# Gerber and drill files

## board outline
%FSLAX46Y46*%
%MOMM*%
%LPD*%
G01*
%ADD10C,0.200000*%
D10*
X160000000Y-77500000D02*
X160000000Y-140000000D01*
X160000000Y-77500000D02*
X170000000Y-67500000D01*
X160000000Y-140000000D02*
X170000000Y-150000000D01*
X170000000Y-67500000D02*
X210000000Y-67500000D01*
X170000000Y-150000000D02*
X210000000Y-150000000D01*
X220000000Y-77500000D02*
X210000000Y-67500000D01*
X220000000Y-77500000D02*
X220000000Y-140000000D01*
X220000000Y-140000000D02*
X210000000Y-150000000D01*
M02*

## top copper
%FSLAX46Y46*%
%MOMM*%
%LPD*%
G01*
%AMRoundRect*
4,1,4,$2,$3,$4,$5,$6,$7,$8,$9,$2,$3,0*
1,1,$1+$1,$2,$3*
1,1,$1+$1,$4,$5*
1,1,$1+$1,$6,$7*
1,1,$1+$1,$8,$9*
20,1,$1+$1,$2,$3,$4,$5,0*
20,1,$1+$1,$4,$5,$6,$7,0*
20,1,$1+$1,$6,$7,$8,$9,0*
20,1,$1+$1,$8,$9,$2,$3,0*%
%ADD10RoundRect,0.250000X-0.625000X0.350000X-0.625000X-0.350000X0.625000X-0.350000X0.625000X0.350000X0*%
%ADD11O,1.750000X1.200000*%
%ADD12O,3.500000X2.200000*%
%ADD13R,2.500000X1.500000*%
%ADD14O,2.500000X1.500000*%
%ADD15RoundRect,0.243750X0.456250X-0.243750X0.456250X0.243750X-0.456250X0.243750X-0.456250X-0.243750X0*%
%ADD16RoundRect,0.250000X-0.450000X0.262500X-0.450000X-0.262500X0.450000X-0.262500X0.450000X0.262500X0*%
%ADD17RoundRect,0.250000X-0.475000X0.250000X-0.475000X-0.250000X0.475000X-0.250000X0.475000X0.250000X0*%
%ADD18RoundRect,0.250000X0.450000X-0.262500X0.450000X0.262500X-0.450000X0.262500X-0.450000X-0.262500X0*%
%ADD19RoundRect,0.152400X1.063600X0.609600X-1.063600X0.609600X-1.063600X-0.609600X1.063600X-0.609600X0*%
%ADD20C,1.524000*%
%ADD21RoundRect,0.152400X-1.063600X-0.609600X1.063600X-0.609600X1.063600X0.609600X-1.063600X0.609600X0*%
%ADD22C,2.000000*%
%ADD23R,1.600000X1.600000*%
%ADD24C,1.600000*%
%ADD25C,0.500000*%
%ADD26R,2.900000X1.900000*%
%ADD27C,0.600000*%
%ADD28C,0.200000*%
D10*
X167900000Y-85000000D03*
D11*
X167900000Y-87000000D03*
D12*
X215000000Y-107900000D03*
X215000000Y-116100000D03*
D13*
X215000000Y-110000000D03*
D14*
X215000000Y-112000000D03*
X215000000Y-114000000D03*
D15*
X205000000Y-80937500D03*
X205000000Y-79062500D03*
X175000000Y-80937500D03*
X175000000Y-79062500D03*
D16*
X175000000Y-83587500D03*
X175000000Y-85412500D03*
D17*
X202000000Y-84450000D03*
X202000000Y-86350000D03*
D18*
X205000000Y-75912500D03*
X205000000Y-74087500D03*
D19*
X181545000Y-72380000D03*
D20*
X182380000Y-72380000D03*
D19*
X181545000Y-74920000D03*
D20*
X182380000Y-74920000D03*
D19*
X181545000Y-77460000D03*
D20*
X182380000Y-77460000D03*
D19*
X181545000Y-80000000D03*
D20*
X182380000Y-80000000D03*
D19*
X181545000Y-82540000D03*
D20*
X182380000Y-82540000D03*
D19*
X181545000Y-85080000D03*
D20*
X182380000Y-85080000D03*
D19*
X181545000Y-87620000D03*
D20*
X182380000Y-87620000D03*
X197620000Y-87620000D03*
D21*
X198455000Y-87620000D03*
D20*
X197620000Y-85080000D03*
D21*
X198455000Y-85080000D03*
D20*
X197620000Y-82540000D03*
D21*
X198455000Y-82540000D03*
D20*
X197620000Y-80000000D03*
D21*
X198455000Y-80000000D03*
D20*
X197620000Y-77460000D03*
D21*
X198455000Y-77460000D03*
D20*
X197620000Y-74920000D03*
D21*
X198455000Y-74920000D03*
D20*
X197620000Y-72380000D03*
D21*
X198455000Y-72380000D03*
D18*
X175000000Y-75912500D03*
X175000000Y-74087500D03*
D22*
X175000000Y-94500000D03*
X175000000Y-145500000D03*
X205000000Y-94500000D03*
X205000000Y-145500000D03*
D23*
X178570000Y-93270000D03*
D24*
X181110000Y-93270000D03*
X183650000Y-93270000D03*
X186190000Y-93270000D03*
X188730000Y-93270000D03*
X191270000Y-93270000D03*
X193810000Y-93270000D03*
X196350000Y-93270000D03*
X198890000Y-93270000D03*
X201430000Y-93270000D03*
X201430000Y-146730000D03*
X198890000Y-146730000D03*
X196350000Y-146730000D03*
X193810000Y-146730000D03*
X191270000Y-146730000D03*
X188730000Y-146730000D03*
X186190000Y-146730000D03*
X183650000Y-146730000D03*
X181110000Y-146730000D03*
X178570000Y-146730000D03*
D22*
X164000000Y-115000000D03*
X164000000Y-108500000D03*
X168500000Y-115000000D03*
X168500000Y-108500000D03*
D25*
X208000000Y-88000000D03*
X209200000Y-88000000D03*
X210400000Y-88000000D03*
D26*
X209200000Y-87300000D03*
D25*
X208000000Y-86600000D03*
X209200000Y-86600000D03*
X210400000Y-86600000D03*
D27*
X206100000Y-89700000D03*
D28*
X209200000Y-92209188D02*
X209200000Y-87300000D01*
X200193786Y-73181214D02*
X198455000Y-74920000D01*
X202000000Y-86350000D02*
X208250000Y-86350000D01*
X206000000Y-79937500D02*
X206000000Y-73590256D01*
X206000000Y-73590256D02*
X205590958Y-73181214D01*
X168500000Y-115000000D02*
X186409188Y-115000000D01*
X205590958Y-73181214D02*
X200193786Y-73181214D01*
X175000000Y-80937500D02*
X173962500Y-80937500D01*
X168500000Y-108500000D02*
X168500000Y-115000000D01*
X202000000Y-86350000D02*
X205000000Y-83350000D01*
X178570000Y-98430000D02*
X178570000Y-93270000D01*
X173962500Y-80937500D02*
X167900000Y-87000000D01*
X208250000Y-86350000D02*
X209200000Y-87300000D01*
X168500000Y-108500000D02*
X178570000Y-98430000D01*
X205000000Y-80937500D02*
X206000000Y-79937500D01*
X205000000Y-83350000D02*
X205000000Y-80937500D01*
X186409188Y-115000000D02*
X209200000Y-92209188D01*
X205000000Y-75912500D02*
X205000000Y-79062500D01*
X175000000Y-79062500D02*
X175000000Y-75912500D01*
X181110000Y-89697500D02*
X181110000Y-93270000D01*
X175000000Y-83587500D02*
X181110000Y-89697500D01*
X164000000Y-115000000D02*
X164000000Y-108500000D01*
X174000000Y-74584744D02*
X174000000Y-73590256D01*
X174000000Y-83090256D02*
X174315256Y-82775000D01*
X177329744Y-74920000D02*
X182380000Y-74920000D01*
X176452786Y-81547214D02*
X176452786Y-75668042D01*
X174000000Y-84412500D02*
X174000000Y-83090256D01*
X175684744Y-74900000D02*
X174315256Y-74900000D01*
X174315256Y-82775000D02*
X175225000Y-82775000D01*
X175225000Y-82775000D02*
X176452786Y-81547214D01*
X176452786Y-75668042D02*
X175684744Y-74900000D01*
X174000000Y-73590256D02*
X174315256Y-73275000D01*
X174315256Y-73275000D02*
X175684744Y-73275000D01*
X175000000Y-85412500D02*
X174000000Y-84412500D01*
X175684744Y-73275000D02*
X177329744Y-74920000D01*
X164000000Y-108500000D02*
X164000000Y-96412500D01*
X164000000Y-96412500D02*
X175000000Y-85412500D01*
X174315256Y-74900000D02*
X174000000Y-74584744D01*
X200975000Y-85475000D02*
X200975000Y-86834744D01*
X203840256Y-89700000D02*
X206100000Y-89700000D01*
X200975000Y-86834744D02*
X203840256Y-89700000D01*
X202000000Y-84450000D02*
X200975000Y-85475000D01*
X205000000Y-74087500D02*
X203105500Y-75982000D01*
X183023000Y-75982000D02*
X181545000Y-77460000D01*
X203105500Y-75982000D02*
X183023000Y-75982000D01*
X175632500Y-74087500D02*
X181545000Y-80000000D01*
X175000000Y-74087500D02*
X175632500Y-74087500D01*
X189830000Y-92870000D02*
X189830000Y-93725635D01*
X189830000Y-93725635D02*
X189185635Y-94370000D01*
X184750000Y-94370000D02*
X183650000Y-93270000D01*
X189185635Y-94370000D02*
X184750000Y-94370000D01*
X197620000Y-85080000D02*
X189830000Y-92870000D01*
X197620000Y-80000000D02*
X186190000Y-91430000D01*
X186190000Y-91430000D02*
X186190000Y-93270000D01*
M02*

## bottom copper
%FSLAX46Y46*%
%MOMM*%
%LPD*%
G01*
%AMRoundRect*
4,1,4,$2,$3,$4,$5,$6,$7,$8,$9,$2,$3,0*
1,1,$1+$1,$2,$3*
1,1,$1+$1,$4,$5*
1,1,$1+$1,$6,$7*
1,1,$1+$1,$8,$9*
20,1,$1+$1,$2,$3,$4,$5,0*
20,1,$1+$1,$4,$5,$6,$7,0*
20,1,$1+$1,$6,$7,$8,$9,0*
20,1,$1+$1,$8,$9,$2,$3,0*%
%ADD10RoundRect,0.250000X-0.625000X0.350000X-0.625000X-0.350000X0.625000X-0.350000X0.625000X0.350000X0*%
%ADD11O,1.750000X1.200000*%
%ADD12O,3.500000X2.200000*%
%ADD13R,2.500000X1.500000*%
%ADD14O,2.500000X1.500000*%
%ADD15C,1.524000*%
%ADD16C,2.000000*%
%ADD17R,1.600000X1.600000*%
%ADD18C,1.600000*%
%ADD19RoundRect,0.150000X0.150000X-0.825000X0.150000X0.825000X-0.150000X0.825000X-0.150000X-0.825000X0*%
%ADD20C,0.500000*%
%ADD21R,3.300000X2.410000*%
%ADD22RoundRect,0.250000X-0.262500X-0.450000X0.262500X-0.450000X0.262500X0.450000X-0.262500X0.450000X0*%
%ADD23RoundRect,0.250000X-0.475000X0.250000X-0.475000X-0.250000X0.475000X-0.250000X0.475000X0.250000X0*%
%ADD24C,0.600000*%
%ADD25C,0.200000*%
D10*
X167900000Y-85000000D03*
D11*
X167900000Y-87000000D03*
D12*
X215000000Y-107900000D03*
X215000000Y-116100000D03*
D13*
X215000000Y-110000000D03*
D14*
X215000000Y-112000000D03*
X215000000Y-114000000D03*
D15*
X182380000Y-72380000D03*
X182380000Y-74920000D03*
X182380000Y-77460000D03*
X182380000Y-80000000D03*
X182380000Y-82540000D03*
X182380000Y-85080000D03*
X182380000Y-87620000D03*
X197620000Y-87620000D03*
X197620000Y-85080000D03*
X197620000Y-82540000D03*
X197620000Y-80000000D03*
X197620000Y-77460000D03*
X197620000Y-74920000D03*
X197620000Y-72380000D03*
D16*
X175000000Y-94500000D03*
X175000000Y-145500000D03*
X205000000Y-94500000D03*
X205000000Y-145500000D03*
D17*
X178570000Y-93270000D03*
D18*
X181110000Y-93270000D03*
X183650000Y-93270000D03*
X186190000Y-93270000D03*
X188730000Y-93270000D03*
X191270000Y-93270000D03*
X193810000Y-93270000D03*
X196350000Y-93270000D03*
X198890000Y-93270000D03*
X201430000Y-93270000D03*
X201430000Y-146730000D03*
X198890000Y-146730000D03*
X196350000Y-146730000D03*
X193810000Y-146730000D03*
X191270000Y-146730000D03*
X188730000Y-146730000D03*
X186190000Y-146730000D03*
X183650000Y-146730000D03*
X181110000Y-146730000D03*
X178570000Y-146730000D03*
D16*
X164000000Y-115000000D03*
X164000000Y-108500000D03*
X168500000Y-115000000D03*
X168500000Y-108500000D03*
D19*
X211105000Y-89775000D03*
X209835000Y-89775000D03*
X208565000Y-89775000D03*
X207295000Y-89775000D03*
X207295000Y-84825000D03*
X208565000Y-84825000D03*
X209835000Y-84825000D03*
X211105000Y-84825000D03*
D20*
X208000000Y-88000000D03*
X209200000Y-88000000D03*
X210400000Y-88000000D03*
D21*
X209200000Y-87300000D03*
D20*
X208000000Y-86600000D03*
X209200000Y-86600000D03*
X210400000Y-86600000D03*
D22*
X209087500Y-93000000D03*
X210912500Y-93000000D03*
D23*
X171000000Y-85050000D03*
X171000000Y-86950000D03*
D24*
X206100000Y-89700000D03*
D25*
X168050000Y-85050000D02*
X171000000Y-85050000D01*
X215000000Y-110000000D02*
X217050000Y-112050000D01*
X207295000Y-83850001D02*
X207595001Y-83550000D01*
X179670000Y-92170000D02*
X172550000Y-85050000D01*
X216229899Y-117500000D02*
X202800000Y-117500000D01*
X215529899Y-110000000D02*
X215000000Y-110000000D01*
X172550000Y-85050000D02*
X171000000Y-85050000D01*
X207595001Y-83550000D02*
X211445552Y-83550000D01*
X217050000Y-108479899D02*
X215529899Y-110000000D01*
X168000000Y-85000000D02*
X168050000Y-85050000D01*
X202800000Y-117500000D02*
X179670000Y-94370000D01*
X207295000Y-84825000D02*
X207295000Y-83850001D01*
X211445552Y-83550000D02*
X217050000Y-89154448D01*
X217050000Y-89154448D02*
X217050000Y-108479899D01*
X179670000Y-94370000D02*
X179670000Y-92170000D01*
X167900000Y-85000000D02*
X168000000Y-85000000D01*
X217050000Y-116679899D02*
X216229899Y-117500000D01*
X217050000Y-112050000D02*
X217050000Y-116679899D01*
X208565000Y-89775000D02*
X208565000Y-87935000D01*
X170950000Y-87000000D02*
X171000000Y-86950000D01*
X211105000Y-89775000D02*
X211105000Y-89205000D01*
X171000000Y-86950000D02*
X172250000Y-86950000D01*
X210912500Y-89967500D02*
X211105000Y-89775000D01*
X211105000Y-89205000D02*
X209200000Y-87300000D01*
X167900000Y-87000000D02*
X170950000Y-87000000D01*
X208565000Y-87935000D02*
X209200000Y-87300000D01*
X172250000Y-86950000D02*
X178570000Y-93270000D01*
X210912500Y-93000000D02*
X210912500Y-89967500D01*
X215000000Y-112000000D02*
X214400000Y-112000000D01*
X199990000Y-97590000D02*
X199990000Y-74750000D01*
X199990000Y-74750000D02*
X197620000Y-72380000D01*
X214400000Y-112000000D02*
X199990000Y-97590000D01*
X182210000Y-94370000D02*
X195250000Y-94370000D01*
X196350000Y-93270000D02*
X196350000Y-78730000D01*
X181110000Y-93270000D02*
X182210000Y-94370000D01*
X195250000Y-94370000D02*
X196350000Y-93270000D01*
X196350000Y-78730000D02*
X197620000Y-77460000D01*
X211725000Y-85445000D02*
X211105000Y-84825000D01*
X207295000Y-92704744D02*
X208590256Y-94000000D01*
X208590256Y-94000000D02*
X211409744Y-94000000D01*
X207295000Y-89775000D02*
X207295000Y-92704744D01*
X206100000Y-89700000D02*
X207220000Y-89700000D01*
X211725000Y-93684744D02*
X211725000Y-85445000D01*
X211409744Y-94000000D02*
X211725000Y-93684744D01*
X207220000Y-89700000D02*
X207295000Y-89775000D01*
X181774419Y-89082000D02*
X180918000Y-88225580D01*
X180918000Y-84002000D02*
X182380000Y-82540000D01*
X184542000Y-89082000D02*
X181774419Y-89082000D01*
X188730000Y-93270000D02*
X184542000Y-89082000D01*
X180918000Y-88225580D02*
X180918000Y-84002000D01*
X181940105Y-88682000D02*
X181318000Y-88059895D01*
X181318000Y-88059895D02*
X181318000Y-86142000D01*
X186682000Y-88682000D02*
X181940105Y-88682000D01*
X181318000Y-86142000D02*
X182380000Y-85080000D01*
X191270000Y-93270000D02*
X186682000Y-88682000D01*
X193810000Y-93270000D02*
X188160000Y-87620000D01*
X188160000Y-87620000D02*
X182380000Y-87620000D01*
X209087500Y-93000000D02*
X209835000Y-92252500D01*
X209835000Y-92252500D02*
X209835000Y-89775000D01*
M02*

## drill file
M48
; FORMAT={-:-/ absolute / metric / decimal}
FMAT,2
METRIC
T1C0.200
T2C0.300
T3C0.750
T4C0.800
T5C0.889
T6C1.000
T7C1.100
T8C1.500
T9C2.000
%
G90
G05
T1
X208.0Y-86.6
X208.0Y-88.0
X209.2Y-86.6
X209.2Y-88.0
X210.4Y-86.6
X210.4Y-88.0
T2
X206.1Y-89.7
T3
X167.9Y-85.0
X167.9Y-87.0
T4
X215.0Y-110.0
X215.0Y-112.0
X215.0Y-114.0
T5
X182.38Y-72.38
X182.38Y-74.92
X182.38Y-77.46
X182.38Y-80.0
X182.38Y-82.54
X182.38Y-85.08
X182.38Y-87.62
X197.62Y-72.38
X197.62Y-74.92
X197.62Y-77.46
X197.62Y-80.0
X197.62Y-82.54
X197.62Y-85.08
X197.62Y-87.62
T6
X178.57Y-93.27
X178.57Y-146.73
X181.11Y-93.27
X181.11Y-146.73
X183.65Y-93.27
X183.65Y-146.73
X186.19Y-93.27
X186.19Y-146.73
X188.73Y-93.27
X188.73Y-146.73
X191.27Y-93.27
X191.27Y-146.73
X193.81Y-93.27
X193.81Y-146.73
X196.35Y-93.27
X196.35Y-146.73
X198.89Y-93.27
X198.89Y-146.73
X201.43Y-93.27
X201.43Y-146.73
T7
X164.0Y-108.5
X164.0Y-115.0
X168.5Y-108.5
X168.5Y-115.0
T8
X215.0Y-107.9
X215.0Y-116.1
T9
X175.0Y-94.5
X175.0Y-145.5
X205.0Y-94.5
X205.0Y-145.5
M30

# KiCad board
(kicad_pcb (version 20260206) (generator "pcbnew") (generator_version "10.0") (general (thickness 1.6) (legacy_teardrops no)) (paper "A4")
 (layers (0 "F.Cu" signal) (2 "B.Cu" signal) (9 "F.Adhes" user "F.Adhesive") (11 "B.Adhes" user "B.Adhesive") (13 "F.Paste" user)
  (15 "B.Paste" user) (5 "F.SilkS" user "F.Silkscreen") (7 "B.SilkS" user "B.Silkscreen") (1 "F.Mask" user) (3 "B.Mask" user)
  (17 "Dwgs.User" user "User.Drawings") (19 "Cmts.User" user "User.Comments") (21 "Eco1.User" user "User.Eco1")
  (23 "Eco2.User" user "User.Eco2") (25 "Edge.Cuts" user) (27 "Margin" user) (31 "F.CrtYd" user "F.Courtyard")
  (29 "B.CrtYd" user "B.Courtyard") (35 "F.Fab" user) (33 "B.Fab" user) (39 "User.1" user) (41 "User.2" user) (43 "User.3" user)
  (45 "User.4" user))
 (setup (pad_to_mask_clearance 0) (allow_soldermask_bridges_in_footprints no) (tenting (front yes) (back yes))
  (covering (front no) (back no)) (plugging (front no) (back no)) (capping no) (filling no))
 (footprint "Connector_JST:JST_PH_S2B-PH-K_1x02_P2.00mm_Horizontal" (layer "F.Cu") (at 167.9 85 -90)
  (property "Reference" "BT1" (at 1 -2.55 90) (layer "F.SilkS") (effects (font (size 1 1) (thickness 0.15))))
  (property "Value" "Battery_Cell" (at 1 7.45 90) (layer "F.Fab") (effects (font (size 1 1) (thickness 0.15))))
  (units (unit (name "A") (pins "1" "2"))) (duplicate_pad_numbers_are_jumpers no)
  (pad "1" thru_hole roundrect (at 0 0 270) (size 1.2 1.75) (drill 0.75) (layers "*.Cu" "*.Mask") (remove_unused_layers no)
   (roundrect_rratio 0.208333) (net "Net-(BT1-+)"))
  (pad "2" thru_hole oval (at 2 0 270) (size 1.2 1.75) (drill 0.75) (layers "*.Cu" "*.Mask") (remove_unused_layers no) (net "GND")))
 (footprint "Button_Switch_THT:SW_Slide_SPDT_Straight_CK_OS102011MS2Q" (layer "F.Cu") (at 215 110 -90)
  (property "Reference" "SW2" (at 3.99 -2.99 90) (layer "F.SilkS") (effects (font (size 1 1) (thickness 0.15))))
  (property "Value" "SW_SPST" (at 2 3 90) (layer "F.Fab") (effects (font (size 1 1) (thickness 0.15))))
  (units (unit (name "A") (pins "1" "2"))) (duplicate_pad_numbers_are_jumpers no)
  (pad "" thru_hole oval (at -2.1 0 270) (size 2.2 3.5) (drill 1.5) (layers "*.Cu" "*.Mask") (remove_unused_layers no))
  (pad "" thru_hole oval (at 6.1 0 270) (size 2.2 3.5) (drill 1.5) (layers "*.Cu" "*.Mask") (remove_unused_layers no))
  (pad "1" thru_hole rect (at 0 0 270) (size 1.5 2.5) (drill 0.8) (layers "*.Cu" "*.Mask") (remove_unused_layers no) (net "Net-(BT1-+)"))
  (pad "2" thru_hole oval (at 2 0 270) (size 1.5 2.5) (drill 0.8) (layers "*.Cu" "*.Mask") (remove_unused_layers no) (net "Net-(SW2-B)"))
  (pad "3" thru_hole oval (at 4 0 270) (size 1.5 2.5) (drill 0.8) (layers "*.Cu" "*.Mask") (remove_unused_layers no)))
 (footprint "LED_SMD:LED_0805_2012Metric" (layer "F.Cu") (at 205 80 90)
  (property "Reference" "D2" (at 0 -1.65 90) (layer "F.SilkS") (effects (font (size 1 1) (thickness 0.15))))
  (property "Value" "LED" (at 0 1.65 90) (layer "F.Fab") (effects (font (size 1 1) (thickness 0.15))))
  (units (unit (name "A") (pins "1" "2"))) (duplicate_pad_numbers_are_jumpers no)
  (pad "1" smd roundrect (at -0.9375 0 90) (size 0.975 1.4) (layers "F.Cu" "F.Mask" "F.Paste") (roundrect_rratio 0.25) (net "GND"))
  (pad "2" smd roundrect (at 0.9375 0 90) (size 0.975 1.4) (layers "F.Cu" "F.Mask" "F.Paste") (roundrect_rratio 0.25) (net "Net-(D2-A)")))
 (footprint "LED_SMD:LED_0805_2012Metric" (layer "F.Cu") (at 175 80 90)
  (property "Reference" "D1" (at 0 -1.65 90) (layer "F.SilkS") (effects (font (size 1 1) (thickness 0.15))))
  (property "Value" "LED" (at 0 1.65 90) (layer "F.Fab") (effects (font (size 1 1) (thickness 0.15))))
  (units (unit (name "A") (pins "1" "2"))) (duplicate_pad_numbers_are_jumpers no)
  (pad "1" smd roundrect (at -0.9375 0 90) (size 0.975 1.4) (layers "F.Cu" "F.Mask" "F.Paste") (roundrect_rratio 0.25) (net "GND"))
  (pad "2" smd roundrect (at 0.9375 0 90) (size 0.975 1.4) (layers "F.Cu" "F.Mask" "F.Paste") (roundrect_rratio 0.25) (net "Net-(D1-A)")))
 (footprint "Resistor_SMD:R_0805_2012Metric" (layer "F.Cu") (at 175 84.5 -90)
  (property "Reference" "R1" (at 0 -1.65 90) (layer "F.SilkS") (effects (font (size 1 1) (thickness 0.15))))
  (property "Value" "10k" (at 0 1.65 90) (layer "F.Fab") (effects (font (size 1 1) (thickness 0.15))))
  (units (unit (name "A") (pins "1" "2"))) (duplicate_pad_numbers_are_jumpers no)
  (pad "1" smd roundrect (at -0.9125 0 270) (size 1.025 1.4) (layers "F.Cu" "F.Mask" "F.Paste") (roundrect_rratio 0.243902) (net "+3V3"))
  (pad "2" smd roundrect (at 0.9125 0 270) (size 1.025 1.4) (layers "F.Cu" "F.Mask" "F.Paste") (roundrect_rratio 0.243902)
   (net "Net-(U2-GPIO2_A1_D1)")))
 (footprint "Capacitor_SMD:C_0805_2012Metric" (layer "F.Cu") (at 202 85.4 -90)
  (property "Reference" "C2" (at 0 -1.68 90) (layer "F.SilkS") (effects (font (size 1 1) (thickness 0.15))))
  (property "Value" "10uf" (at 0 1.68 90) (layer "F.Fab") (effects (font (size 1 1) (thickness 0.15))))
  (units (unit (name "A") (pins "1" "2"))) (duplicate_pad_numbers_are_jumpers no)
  (pad "1" smd roundrect (at -0.95 0 270) (size 1 1.45) (layers "F.Cu" "F.Mask" "F.Paste") (roundrect_rratio 0.25) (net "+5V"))
  (pad "2" smd roundrect (at 0.95 0 270) (size 1 1.45) (layers "F.Cu" "F.Mask" "F.Paste") (roundrect_rratio 0.25) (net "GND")))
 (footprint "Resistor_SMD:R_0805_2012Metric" (layer "F.Cu") (at 205 75 90)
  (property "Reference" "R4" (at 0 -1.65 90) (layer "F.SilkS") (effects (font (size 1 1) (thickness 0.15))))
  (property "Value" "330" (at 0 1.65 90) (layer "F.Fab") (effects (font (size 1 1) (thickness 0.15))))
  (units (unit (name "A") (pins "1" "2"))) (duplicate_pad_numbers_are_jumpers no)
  (pad "1" smd roundrect (at -0.9125 0 90) (size 1.025 1.4) (layers "F.Cu" "F.Mask" "F.Paste") (roundrect_rratio 0.243902)
   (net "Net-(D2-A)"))
  (pad "2" smd roundrect (at 0.9125 0 90) (size 1.025 1.4) (layers "F.Cu" "F.Mask" "F.Paste") (roundrect_rratio 0.243902)
   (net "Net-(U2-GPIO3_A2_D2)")))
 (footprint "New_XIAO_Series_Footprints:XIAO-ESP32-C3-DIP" (layer "F.Cu") (at 190 80 90)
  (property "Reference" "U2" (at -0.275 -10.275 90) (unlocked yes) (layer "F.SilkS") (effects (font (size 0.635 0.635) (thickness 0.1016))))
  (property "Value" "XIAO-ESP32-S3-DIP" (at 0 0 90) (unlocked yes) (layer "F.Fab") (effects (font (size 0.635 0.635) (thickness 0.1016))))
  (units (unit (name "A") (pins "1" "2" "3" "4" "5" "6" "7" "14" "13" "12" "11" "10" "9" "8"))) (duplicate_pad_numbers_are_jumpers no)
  (pad "1" smd roundrect (at 7.62 -8.455 180) (size 2.432 1.524) (layers "F.Cu" "F.Mask") (roundrect_rratio 0.1)
   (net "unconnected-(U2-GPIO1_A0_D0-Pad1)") (thermal_bridge_angle 45))
  (pad "1" thru_hole circle (at 7.62 -7.62 180) (size 1.524 1.524) (drill 0.889) (layers "*.Cu" "*.Mask") (remove_unused_layers no)
   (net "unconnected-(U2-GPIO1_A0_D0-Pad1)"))
  (pad "2" smd roundrect (at 5.08 -8.455 180) (size 2.432 1.524) (layers "F.Cu" "F.Mask") (roundrect_rratio 0.1)
   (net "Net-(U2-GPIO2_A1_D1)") (thermal_bridge_angle 45))
  (pad "2" thru_hole circle (at 5.08 -7.62 180) (size 1.524 1.524) (drill 0.889) (layers "*.Cu" "*.Mask") (remove_unused_layers no)
   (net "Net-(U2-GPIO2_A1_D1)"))
  (pad "3" smd roundrect (at 2.54 -8.455 180) (size 2.432 1.524) (layers "F.Cu" "F.Mask") (roundrect_rratio 0.1)
   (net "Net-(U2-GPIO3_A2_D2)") (thermal_bridge_angle 45))
  (pad "3" thru_hole circle (at 2.54 -7.62 180) (size 1.524 1.524) (drill 0.889) (layers "*.Cu" "*.Mask") (remove_unused_layers no)
   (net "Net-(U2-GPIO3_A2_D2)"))
  (pad "4" smd roundrect (at 0 -8.455 180) (size 2.432 1.524) (layers "F.Cu" "F.Mask") (roundrect_rratio 0.1) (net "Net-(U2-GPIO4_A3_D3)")
   (thermal_bridge_angle 45))
  (pad "4" thru_hole circle (at 0 -7.62 180) (size 1.524 1.524) (drill 0.889) (layers "*.Cu" "*.Mask") (remove_unused_layers no)
   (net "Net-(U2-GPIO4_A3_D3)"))
  (pad "5" smd roundrect (at -2.54 -8.455 180) (size 2.432 1.524) (layers "F.Cu" "F.Mask") (roundrect_rratio 0.1) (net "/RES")
   (thermal_bridge_angle 45))
  (pad "5" thru_hole circle (at -2.54 -7.62 180) (size 1.524 1.524) (drill 0.889) (layers "*.Cu" "*.Mask") (remove_unused_layers no)
   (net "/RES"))
  (pad "6" smd roundrect (at -5.08 -8.455 180) (size 2.432 1.524) (layers "F.Cu" "F.Mask") (roundrect_rratio 0.1) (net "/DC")
   (thermal_bridge_angle 45))
  (pad "6" thru_hole circle (at -5.08 -7.62 180) (size 1.524 1.524) (drill 0.889) (layers "*.Cu" "*.Mask") (remove_unused_layers no)
   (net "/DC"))
  (pad "7" smd roundrect (at -7.62 -8.455 180) (size 2.432 1.524) (layers "F.Cu" "F.Mask") (roundrect_rratio 0.1) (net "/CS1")
   (thermal_bridge_angle 45))
  (pad "7" thru_hole circle (at -7.62 -7.62 180) (size 1.524 1.524) (drill 0.889) (layers "*.Cu" "*.Mask") (remove_unused_layers no)
   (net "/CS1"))
  (pad "8" thru_hole circle (at -7.62 7.62) (size 1.524 1.524) (drill 0.889) (layers "*.Cu" "*.Mask") (remove_unused_layers no)
   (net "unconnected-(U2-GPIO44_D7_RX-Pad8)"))
  (pad "8" smd roundrect (at -7.62 8.455) (size 2.432 1.524) (layers "F.Cu" "F.Mask") (roundrect_rratio 0.1)
   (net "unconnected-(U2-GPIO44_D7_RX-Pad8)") (thermal_bridge_angle 45))
  (pad "9" thru_hole circle (at -5.08 7.62) (size 1.524 1.524) (drill 0.889) (layers "*.Cu" "*.Mask") (remove_unused_layers no)
   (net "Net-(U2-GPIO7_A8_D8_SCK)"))
  (pad "9" smd roundrect (at -5.08 8.455) (size 2.432 1.524) (layers "F.Cu" "F.Mask") (roundrect_rratio 0.1)
   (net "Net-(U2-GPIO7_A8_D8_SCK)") (thermal_bridge_angle 45))
  (pad "10" thru_hole circle (at -2.54 7.62) (size 1.524 1.524) (drill 0.889) (layers "*.Cu" "*.Mask") (remove_unused_layers no)
   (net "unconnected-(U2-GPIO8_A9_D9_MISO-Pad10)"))
  (pad "10" smd roundrect (at -2.54 8.455) (size 2.432 1.524) (layers "F.Cu" "F.Mask") (roundrect_rratio 0.1)
   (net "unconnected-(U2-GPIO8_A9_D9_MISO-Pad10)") (thermal_bridge_angle 45))
  (pad "11" thru_hole circle (at 0 7.62) (size 1.524 1.524) (drill 0.889) (layers "*.Cu" "*.Mask") (remove_unused_layers no)
   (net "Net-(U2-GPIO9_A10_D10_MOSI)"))
  (pad "11" smd roundrect (at 0 8.455) (size 2.432 1.524) (layers "F.Cu" "F.Mask") (roundrect_rratio 0.1)
   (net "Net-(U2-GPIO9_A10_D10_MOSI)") (thermal_bridge_angle 45))
  (pad "12" thru_hole circle (at 2.54 7.62) (size 1.524 1.524) (drill 0.889) (layers "*.Cu" "*.Mask") (remove_unused_layers no) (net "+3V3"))
  (pad "12" smd roundrect (at 2.54 8.455) (size 2.432 1.524) (layers "F.Cu" "F.Mask") (roundrect_rratio 0.1) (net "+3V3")
   (thermal_bridge_angle 45))
  (pad "13" thru_hole circle (at 5.08 7.62) (size 1.524 1.524) (drill 0.889) (layers "*.Cu" "*.Mask") (remove_unused_layers no) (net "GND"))
  (pad "13" smd roundrect (at 5.08 8.455) (size 2.432 1.524) (layers "F.Cu" "F.Mask") (roundrect_rratio 0.1) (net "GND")
   (thermal_bridge_angle 45))
  (pad "14" thru_hole circle (at 7.62 7.62) (size 1.524 1.524) (drill 0.889) (layers "*.Cu" "*.Mask") (remove_unused_layers no)
   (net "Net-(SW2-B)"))
  (pad "14" smd roundrect (at 7.62 8.455) (size 2.432 1.524) (layers "F.Cu" "F.Mask") (roundrect_rratio 0.1) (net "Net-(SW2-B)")
   (thermal_bridge_angle 45)))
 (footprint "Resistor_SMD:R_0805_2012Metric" (layer "F.Cu") (at 175 75 90)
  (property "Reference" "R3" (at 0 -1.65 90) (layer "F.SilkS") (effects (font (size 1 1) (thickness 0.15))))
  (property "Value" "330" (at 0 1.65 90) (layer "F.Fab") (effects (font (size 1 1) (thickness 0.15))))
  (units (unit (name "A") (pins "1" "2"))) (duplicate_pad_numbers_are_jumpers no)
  (pad "1" smd roundrect (at -0.9125 0 90) (size 1.025 1.4) (layers "F.Cu" "F.Mask" "F.Paste") (roundrect_rratio 0.243902)
   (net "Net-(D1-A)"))
  (pad "2" smd roundrect (at 0.9125 0 90) (size 1.025 1.4) (layers "F.Cu" "F.Mask" "F.Paste") (roundrect_rratio 0.243902)
   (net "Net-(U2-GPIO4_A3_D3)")))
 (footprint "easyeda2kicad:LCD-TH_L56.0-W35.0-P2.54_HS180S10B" (layer "F.Cu") (at 190 120)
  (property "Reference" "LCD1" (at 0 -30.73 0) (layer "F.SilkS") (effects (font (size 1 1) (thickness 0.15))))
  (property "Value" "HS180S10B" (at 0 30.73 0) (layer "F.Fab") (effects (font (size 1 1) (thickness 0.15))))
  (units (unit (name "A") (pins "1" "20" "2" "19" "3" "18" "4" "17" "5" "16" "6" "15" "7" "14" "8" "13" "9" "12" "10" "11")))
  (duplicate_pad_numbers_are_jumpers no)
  (pad "" thru_hole circle (at -15 -25.5) (size 2 2) (drill 2) (layers "*.Cu" "*.Mask") (remove_unused_layers no))
  (pad "" thru_hole circle (at -15 25.5) (size 2 2) (drill 2) (layers "*.Cu" "*.Mask") (remove_unused_layers no))
  (pad "" thru_hole circle (at 15 -25.5) (size 2 2) (drill 2) (layers "*.Cu" "*.Mask") (remove_unused_layers no))
  (pad "" thru_hole circle (at 15 25.5) (size 2 2) (drill 2) (layers "*.Cu" "*.Mask") (remove_unused_layers no))
  (pad "1" thru_hole rect (at -11.43 -26.73) (size 1.6 1.6) (drill 0.999998) (layers "*.Cu" "*.Mask") (remove_unused_layers no) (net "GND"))
  (pad "2" thru_hole circle (at -8.89 -26.73) (size 1.6 1.6) (drill 0.999998) (layers "*.Cu" "*.Mask") (remove_unused_layers no)
   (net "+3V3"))
  (pad "3" thru_hole circle (at -6.35 -26.73) (size 1.6 1.6) (drill 0.999998) (layers "*.Cu" "*.Mask") (remove_unused_layers no)
   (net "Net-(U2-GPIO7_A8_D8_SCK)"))
  (pad "4" thru_hole circle (at -3.81 -26.73) (size 1.6 1.6) (drill 0.999998) (layers "*.Cu" "*.Mask") (remove_unused_layers no)
   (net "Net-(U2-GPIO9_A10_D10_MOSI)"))
  (pad "5" thru_hole circle (at -1.27 -26.73) (size 1.6 1.6) (drill 0.999998) (layers "*.Cu" "*.Mask") (remove_unused_layers no)
   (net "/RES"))
  (pad "6" thru_hole circle (at 1.27 -26.73) (size 1.6 1.6) (drill 0.999998) (layers "*.Cu" "*.Mask") (remove_unused_layers no) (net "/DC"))
  (pad "7" thru_hole circle (at 3.81 -26.73) (size 1.6 1.6) (drill 0.999998) (layers "*.Cu" "*.Mask") (remove_unused_layers no) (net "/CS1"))
  (pad "8" thru_hole circle (at 6.35 -26.73) (size 1.6 1.6) (drill 0.999998) (layers "*.Cu" "*.Mask") (remove_unused_layers no) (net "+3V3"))
  (pad "9" thru_hole circle (at 8.89 -26.73) (size 1.6 1.6) (drill 0.999998) (layers "*.Cu" "*.Mask") (remove_unused_layers no)
   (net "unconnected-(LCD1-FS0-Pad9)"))
  (pad "10" thru_hole circle (at 11.43 -26.73) (size 1.6 1.6) (drill 0.999998) (layers "*.Cu" "*.Mask") (remove_unused_layers no)
   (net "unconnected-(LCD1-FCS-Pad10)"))
  (pad "11" thru_hole circle (at 11.43 26.73) (size 1.6 1.6) (drill 0.999998) (layers "*.Cu" "*.Mask") (remove_unused_layers no)
   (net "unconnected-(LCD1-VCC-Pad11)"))
  (pad "12" thru_hole circle (at 8.89 26.73) (size 1.6 1.6) (drill 0.999998) (layers "*.Cu" "*.Mask") (remove_unused_layers no)
   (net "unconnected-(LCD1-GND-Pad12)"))
  (pad "13" thru_hole circle (at 6.35 26.73) (size 1.6 1.6) (drill 0.999998) (layers "*.Cu" "*.Mask") (remove_unused_layers no)
   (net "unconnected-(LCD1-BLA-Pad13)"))
  (pad "14" thru_hole circle (at 3.81 26.73) (size 1.6 1.6) (drill 0.999998) (layers "*.Cu" "*.Mask") (remove_unused_layers no)
   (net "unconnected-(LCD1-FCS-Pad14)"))
  (pad "15" thru_hole circle (at 1.27 26.73) (size 1.6 1.6) (drill 0.999998) (layers "*.Cu" "*.Mask") (remove_unused_layers no)
   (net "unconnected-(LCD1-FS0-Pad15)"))
  (pad "16" thru_hole circle (at -1.27 26.73) (size 1.6 1.6) (drill 0.999998) (layers "*.Cu" "*.Mask") (remove_unused_layers no)
   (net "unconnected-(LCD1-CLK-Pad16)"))
  (pad "17" thru_hole circle (at -3.81 26.73) (size 1.6 1.6) (drill 0.999998) (layers "*.Cu" "*.Mask") (remove_unused_layers no)
   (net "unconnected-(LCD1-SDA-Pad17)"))
  (pad "18" thru_hole circle (at -6.35 26.73) (size 1.6 1.6) (drill 0.999998) (layers "*.Cu" "*.Mask") (remove_unused_layers no)
   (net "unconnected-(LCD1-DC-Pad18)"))
  (pad "19" thru_hole circle (at -8.89 26.73) (size 1.6 1.6) (drill 0.999998) (layers "*.Cu" "*.Mask") (remove_unused_layers no)
   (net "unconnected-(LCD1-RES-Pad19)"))
  (pad "20" thru_hole circle (at -11.43 26.73) (size 1.6 1.6) (drill 0.999998) (layers "*.Cu" "*.Mask") (remove_unused_layers no)
   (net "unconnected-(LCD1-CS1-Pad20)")))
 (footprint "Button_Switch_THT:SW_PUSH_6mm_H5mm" (layer "F.Cu") (at 164 115 90)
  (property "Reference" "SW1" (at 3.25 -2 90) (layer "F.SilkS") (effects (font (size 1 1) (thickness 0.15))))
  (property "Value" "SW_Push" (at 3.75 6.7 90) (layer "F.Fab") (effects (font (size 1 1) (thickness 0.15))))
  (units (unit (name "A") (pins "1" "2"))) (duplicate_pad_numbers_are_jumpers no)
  (pad "1" thru_hole circle (at 0 0 180) (size 2 2) (drill 1.1) (layers "*.Cu" "*.Mask") (remove_unused_layers no)
   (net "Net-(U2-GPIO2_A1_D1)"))
  (pad "1" thru_hole circle (at 6.5 0 180) (size 2 2) (drill 1.1) (layers "*.Cu" "*.Mask") (remove_unused_layers no)
   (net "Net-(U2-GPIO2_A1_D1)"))
  (pad "2" thru_hole circle (at 0 4.5 180) (size 2 2) (drill 1.1) (layers "*.Cu" "*.Mask") (remove_unused_layers no) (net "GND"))
  (pad "2" thru_hole circle (at 6.5 4.5 180) (size 2 2) (drill 1.1) (layers "*.Cu" "*.Mask") (remove_unused_layers no) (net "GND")))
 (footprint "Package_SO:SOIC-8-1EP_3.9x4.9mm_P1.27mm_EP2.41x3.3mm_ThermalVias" (layer "B.Cu") (at 209.2 87.3 90)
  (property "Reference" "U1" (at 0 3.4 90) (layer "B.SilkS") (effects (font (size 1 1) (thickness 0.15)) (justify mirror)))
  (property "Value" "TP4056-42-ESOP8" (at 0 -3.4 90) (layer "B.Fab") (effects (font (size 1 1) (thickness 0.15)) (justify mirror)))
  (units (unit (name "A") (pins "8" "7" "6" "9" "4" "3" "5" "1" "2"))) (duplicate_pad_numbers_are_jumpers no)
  (pad "" smd roundrect (at -0.6 -0.825 90) (size 1.01 1.38) (layers "B.Paste") (roundrect_rratio 0.247525))
  (pad "" smd roundrect (at -0.6 0.825 90) (size 1.01 1.38) (layers "B.Paste") (roundrect_rratio 0.247525))
  (pad "" smd roundrect (at 0.6 -0.825 90) (size 1.01 1.38) (layers "B.Paste") (roundrect_rratio 0.247525))
  (pad "" smd roundrect (at 0.6 0.825 90) (size 1.01 1.38) (layers "B.Paste") (roundrect_rratio 0.247525))
  (pad "1" smd roundrect (at -2.475 1.905 90) (size 1.95 0.6) (layers "B.Cu" "B.Mask" "B.Paste") (roundrect_rratio 0.25) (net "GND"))
  (pad "2" smd roundrect (at -2.475 0.635 90) (size 1.95 0.6) (layers "B.Cu" "B.Mask" "B.Paste") (roundrect_rratio 0.25)
   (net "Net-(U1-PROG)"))
  (pad "3" smd roundrect (at -2.475 -0.635 90) (size 1.95 0.6) (layers "B.Cu" "B.Mask" "B.Paste") (roundrect_rratio 0.25) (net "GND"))
  (pad "4" smd roundrect (at -2.475 -1.905 90) (size 1.95 0.6) (layers "B.Cu" "B.Mask" "B.Paste") (roundrect_rratio 0.25) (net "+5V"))
  (pad "5" smd roundrect (at 2.475 -1.905 90) (size 1.95 0.6) (layers "B.Cu" "B.Mask" "B.Paste") (roundrect_rratio 0.25) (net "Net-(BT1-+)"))
  (pad "6" smd roundrect (at 2.475 -0.635 90) (size 1.95 0.6) (layers "B.Cu" "B.Mask" "B.Paste") (roundrect_rratio 0.25)
   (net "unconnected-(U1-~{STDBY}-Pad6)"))
  (pad "7" smd roundrect (at 2.475 0.635 90) (size 1.95 0.6) (layers "B.Cu" "B.Mask" "B.Paste") (roundrect_rratio 0.25)
   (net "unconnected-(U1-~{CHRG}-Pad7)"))
  (pad "8" smd roundrect (at 2.475 1.905 90) (size 1.95 0.6) (layers "B.Cu" "B.Mask" "B.Paste") (roundrect_rratio 0.25) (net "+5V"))
  (pad "9" thru_hole circle (at -0.7 -1.2 90) (size 0.5 0.5) (drill 0.2) (layers "*.Cu") (remove_unused_layers no) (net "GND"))
  (pad "9" thru_hole circle (at -0.7 0 90) (size 0.5 0.5) (drill 0.2) (layers "*.Cu") (remove_unused_layers no) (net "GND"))
  (pad "9" thru_hole circle (at -0.7 1.2 90) (size 0.5 0.5) (drill 0.2) (layers "*.Cu") (remove_unused_layers no) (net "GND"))
  (pad "9" smd rect (at 0 0 90) (size 1.9 2.9) (layers "F.Cu") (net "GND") (zone_connect 2))
  (pad "9" smd rect (at 0 0 90) (size 2.41 3.3) (layers "B.Cu" "B.Mask") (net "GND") (zone_connect 2))
  (pad "9" thru_hole circle (at 0.7 -1.2 90) (size 0.5 0.5) (drill 0.2) (layers "*.Cu") (remove_unused_layers no) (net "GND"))
  (pad "9" thru_hole circle (at 0.7 0 90) (size 0.5 0.5) (drill 0.2) (layers "*.Cu") (remove_unused_layers no) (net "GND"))
  (pad "9" thru_hole circle (at 0.7 1.2 90) (size 0.5 0.5) (drill 0.2) (layers "*.Cu") (remove_unused_layers no) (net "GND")))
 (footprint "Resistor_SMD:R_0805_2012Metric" (layer "B.Cu") (at 210 93)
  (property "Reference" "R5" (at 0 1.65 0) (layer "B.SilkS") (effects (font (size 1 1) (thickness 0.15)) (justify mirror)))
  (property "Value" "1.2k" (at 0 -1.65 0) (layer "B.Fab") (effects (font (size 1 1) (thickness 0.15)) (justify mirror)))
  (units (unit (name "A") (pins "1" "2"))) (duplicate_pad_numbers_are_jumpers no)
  (pad "1" smd roundrect (at -0.9125 0) (size 1.025 1.4) (layers "B.Cu" "B.Mask" "B.Paste") (roundrect_rratio 0.243902)
   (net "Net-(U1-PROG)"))
  (pad "2" smd roundrect (at 0.9125 0) (size 1.025 1.4) (layers "B.Cu" "B.Mask" "B.Paste") (roundrect_rratio 0.243902) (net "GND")))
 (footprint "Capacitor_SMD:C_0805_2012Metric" (layer "B.Cu") (at 171 86 -90)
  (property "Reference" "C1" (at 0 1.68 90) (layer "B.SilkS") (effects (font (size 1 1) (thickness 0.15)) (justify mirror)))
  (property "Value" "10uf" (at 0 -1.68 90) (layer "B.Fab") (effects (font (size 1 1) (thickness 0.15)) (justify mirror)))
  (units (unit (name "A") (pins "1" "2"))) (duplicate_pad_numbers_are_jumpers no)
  (pad "1" smd roundrect (at -0.95 0 270) (size 1 1.45) (layers "B.Cu" "B.Mask" "B.Paste") (roundrect_rratio 0.25) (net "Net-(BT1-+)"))
  (pad "2" smd roundrect (at 0.95 0 270) (size 1 1.45) (layers "B.Cu" "B.Mask" "B.Paste") (roundrect_rratio 0.25) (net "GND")))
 (gr_line (start 160 77.5) (end 160 140) (stroke (width 0.2) (type default)) (layer "Edge.Cuts"))
 (gr_line (start 160 77.5) (end 170 67.5) (stroke (width 0.2) (type default)) (layer "Edge.Cuts"))
 (gr_line (start 160 140) (end 170 150) (stroke (width 0.2) (type default)) (layer "Edge.Cuts"))
 (gr_line (start 170 67.5) (end 210 67.5) (stroke (width 0.2) (type default)) (layer "Edge.Cuts"))
 (gr_line (start 170 150) (end 210 150) (stroke (width 0.2) (type default)) (layer "Edge.Cuts"))
 (gr_line (start 220 77.5) (end 210 67.5) (stroke (width 0.2) (type default)) (layer "Edge.Cuts"))
 (gr_line (start 220 77.5) (end 220 140) (stroke (width 0.2) (type default)) (layer "Edge.Cuts"))
 (gr_line (start 220 140) (end 210 150) (stroke (width 0.2) (type default)) (layer "Edge.Cuts"))
 (segment (start 168.05 85.05) (end 171 85.05) (width 0.2) (layer "B.Cu") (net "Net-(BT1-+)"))
 (segment (start 215 110) (end 217.05 112.05) (width 0.2) (layer "B.Cu") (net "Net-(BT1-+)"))
 (segment (start 207.295 83.850001) (end 207.595001 83.55) (width 0.2) (layer "B.Cu") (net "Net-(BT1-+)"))
 (segment (start 179.67 92.17) (end 172.55 85.05) (width 0.2) (layer "B.Cu") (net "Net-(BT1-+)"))
 (segment (start 216.229899 117.5) (end 202.8 117.5) (width 0.2) (layer "B.Cu") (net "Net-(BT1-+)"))
 (segment (start 215.529899 110) (end 215 110) (width 0.2) (layer "B.Cu") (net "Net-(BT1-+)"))
 (segment (start 172.55 85.05) (end 171 85.05) (width 0.2) (layer "B.Cu") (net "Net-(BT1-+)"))
 (segment (start 207.595001 83.55) (end 211.445552 83.55) (width 0.2) (layer "B.Cu") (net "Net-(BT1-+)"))
 (segment (start 217.05 108.479899) (end 215.529899 110) (width 0.2) (layer "B.Cu") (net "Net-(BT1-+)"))
 (segment (start 168 85) (end 168.05 85.05) (width 0.2) (layer "B.Cu") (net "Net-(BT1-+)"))
 (segment (start 202.8 117.5) (end 179.67 94.37) (width 0.2) (layer "B.Cu") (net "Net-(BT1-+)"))
 (segment (start 207.295 84.825) (end 207.295 83.850001) (width 0.2) (layer "B.Cu") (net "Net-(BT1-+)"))
 (segment (start 211.445552 83.55) (end 217.05 89.154448) (width 0.2) (layer "B.Cu") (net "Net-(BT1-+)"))
 (segment (start 217.05 89.154448) (end 217.05 108.479899) (width 0.2) (layer "B.Cu") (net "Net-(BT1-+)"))
 (segment (start 179.67 94.37) (end 179.67 92.17) (width 0.2) (layer "B.Cu") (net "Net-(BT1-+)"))
 (segment (start 167.9 85) (end 168 85) (width 0.2) (layer "B.Cu") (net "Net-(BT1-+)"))
 (segment (start 217.05 116.679899) (end 216.229899 117.5) (width 0.2) (layer "B.Cu") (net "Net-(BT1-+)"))
 (segment (start 217.05 112.05) (end 217.05 116.679899) (width 0.2) (layer "B.Cu") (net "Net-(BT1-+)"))
 (segment (start 209.2 92.209188) (end 209.2 87.3) (width 0.2) (layer "F.Cu") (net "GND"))
 (segment (start 200.193786 73.181214) (end 198.455 74.92) (width 0.2) (layer "F.Cu") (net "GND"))
 (segment (start 202 86.35) (end 208.25 86.35) (width 0.2) (layer "F.Cu") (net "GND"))
 (segment (start 206 79.9375) (end 206 73.590256) (width 0.2) (layer "F.Cu") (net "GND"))
 (segment (start 206 73.590256) (end 205.590958 73.181214) (width 0.2) (layer "F.Cu") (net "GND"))
 (segment (start 168.5 115) (end 186.409188 115) (width 0.2) (layer "F.Cu") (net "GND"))
 (segment (start 205.590958 73.181214) (end 200.193786 73.181214) (width 0.2) (layer "F.Cu") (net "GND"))
 (segment (start 175 80.9375) (end 173.9625 80.9375) (width 0.2) (layer "F.Cu") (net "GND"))
 (segment (start 168.5 108.5) (end 168.5 115) (width 0.2) (layer "F.Cu") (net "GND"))
 (segment (start 202 86.35) (end 205 83.35) (width 0.2) (layer "F.Cu") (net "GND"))
 (segment (start 178.57 98.43) (end 178.57 93.27) (width 0.2) (layer "F.Cu") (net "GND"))
 (segment (start 173.9625 80.9375) (end 167.9 87) (width 0.2) (layer "F.Cu") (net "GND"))
 (segment (start 208.25 86.35) (end 209.2 87.3) (width 0.2) (layer "F.Cu") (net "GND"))
 (segment (start 168.5 108.5) (end 178.57 98.43) (width 0.2) (layer "F.Cu") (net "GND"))
 (segment (start 205 80.9375) (end 206 79.9375) (width 0.2) (layer "F.Cu") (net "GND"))
 (segment (start 205 83.35) (end 205 80.9375) (width 0.2) (layer "F.Cu") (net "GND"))
 (segment (start 186.409188 115) (end 209.2 92.209188) (width 0.2) (layer "F.Cu") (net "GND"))
 (segment (start 208.565 89.775) (end 208.565 87.935) (width 0.2) (layer "B.Cu") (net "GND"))
 (segment (start 170.95 87) (end 171 86.95) (width 0.2) (layer "B.Cu") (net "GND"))
 (segment (start 211.105 89.775) (end 211.105 89.205) (width 0.2) (layer "B.Cu") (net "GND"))
 (segment (start 171 86.95) (end 172.25 86.95) (width 0.2) (layer "B.Cu") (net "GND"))
 (segment (start 210.9125 89.9675) (end 211.105 89.775) (width 0.2) (layer "B.Cu") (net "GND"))
 (segment (start 211.105 89.205) (end 209.2 87.3) (width 0.2) (layer "B.Cu") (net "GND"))
 (segment (start 167.9 87) (end 170.95 87) (width 0.2) (layer "B.Cu") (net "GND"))
 (segment (start 208.565 87.935) (end 209.2 87.3) (width 0.2) (layer "B.Cu") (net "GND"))
 (segment (start 172.25 86.95) (end 178.57 93.27) (width 0.2) (layer "B.Cu") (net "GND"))
 (segment (start 210.9125 93) (end 210.9125 89.9675) (width 0.2) (layer "B.Cu") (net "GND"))
 (segment (start 215 112) (end 214.4 112) (width 0.2) (layer "B.Cu") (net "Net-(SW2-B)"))
 (segment (start 199.99 97.59) (end 199.99 74.75) (width 0.2) (layer "B.Cu") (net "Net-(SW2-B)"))
 (segment (start 199.99 74.75) (end 197.62 72.38) (width 0.2) (layer "B.Cu") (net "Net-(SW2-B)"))
 (segment (start 214.4 112) (end 199.99 97.59) (width 0.2) (layer "B.Cu") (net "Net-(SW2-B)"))
 (segment (start 205 75.9125) (end 205 79.0625) (width 0.2) (layer "F.Cu") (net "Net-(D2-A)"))
 (segment (start 175 79.0625) (end 175 75.9125) (width 0.2) (layer "F.Cu") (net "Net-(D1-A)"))
 (segment (start 181.11 89.6975) (end 181.11 93.27) (width 0.2) (layer "F.Cu") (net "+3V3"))
 (segment (start 175 83.5875) (end 181.11 89.6975) (width 0.2) (layer "F.Cu") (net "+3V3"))
 (segment (start 182.21 94.37) (end 195.25 94.37) (width 0.2) (layer "B.Cu") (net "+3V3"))
 (segment (start 196.35 93.27) (end 196.35 78.73) (width 0.2) (layer "B.Cu") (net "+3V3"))
 (segment (start 181.11 93.27) (end 182.21 94.37) (width 0.2) (layer "B.Cu") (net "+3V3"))
 (segment (start 195.25 94.37) (end 196.35 93.27) (width 0.2) (layer "B.Cu") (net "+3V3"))
 (segment (start 196.35 78.73) (end 197.62 77.46) (width 0.2) (layer "B.Cu") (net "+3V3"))
 (segment (start 164 115) (end 164 108.5) (width 0.2) (layer "F.Cu") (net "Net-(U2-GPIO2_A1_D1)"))
 (segment (start 174 74.584744) (end 174 73.590256) (width 0.2) (layer "F.Cu") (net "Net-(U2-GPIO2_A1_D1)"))
 (segment (start 174 83.090256) (end 174.315256 82.775) (width 0.2) (layer "F.Cu") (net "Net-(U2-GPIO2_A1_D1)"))
 (segment (start 177.329744 74.92) (end 182.38 74.92) (width 0.2) (layer "F.Cu") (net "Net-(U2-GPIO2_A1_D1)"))
 (segment (start 176.452786 81.547214) (end 176.452786 75.668042) (width 0.2) (layer "F.Cu") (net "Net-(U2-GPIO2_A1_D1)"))
 (segment (start 174 84.4125) (end 174 83.090256) (width 0.2) (layer "F.Cu") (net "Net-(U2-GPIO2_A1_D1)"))
 (segment (start 175.684744 74.9) (end 174.315256 74.9) (width 0.2) (layer "F.Cu") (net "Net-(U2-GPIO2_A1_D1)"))
 (segment (start 174.315256 82.775) (end 175.225 82.775) (width 0.2) (layer "F.Cu") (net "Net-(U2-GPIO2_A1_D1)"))
 (segment (start 175.225 82.775) (end 176.452786 81.547214) (width 0.2) (layer "F.Cu") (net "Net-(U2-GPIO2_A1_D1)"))
 (segment (start 176.452786 75.668042) (end 175.684744 74.9) (width 0.2) (layer "F.Cu") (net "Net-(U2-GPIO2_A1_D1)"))
 (segment (start 174 73.590256) (end 174.315256 73.275) (width 0.2) (layer "F.Cu") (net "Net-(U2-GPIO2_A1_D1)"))
 (segment (start 174.315256 73.275) (end 175.684744 73.275) (width 0.2) (layer "F.Cu") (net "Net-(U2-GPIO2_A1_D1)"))
 (segment (start 175 85.4125) (end 174 84.4125) (width 0.2) (layer "F.Cu") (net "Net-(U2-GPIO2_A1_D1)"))
 (segment (start 175.684744 73.275) (end 177.329744 74.92) (width 0.2) (layer "F.Cu") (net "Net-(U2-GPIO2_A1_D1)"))
 (segment (start 164 108.5) (end 164 96.4125) (width 0.2) (layer "F.Cu") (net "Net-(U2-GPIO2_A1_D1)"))
 (segment (start 164 96.4125) (end 175 85.4125) (width 0.2) (layer "F.Cu") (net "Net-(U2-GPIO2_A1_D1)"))
 (segment (start 174.315256 74.9) (end 174 74.584744) (width 0.2) (layer "F.Cu") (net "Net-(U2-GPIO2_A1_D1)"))
 (segment (start 200.975 85.475) (end 200.975 86.834744) (width 0.2) (layer "F.Cu") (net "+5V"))
 (segment (start 203.840256 89.7) (end 206.1 89.7) (width 0.2) (layer "F.Cu") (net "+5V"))
 (segment (start 200.975 86.834744) (end 203.840256 89.7) (width 0.2) (layer "F.Cu") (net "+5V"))
 (segment (start 202 84.45) (end 200.975 85.475) (width 0.2) (layer "F.Cu") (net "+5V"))
 (via (at 206.1 89.7) (size 0.6) (drill 0.3) (layers "F.Cu" "B.Cu") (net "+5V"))
 (segment (start 211.725 85.445) (end 211.105 84.825) (width 0.2) (layer "B.Cu") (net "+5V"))
 (segment (start 207.295 92.704744) (end 208.590256 94) (width 0.2) (layer "B.Cu") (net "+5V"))
 (segment (start 208.590256 94) (end 211.409744 94) (width 0.2) (layer "B.Cu") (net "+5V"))
 (segment (start 207.295 89.775) (end 207.295 92.704744) (width 0.2) (layer "B.Cu") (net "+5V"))
 (segment (start 206.1 89.7) (end 207.22 89.7) (width 0.2) (layer "B.Cu") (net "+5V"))
 (segment (start 211.725 93.684744) (end 211.725 85.445) (width 0.2) (layer "B.Cu") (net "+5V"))
 (segment (start 211.409744 94) (end 211.725 93.684744) (width 0.2) (layer "B.Cu") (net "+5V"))
 (segment (start 207.22 89.7) (end 207.295 89.775) (width 0.2) (layer "B.Cu") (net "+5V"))
 (segment (start 205 74.0875) (end 203.1055 75.982) (width 0.2) (layer "F.Cu") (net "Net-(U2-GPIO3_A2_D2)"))
 (segment (start 183.023 75.982) (end 181.545 77.46) (width 0.2) (layer "F.Cu") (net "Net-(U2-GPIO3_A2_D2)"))
 (segment (start 203.1055 75.982) (end 183.023 75.982) (width 0.2) (layer "F.Cu") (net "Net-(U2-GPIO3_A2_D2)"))
 (segment (start 175.6325 74.0875) (end 181.545 80) (width 0.2) (layer "F.Cu") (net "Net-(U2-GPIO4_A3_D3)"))
 (segment (start 175 74.0875) (end 175.6325 74.0875) (width 0.2) (layer "F.Cu") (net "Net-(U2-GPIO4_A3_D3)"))
 (segment (start 181.774419 89.082) (end 180.918 88.22558) (width 0.2) (layer "B.Cu") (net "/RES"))
 (segment (start 180.918 84.002) (end 182.38 82.54) (width 0.2) (layer "B.Cu") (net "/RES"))
 (segment (start 184.542 89.082) (end 181.774419 89.082) (width 0.2) (layer "B.Cu") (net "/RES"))
 (segment (start 188.73 93.27) (end 184.542 89.082) (width 0.2) (layer "B.Cu") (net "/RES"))
 (segment (start 180.918 88.22558) (end 180.918 84.002) (width 0.2) (layer "B.Cu") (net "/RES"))
 (segment (start 181.940105 88.682) (end 181.318 88.059895) (width 0.2) (layer "B.Cu") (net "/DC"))
 (segment (start 181.318 88.059895) (end 181.318 86.142) (width 0.2) (layer "B.Cu") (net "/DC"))
 (segment (start 186.682 88.682) (end 181.940105 88.682) (width 0.2) (layer "B.Cu") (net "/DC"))
 (segment (start 181.318 86.142) (end 182.38 85.08) (width 0.2) (layer "B.Cu") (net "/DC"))
 (segment (start 191.27 93.27) (end 186.682 88.682) (width 0.2) (layer "B.Cu") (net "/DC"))
 (segment (start 193.81 93.27) (end 188.16 87.62) (width 0.2) (layer "B.Cu") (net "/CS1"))
 (segment (start 188.16 87.62) (end 182.38 87.62) (width 0.2) (layer "B.Cu") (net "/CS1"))
 (segment (start 189.83 92.87) (end 189.83 93.725635) (width 0.2) (layer "F.Cu") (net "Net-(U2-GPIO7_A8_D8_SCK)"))
 (segment (start 189.83 93.725635) (end 189.185635 94.37) (width 0.2) (layer "F.Cu") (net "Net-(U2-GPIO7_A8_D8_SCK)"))
 (segment (start 184.75 94.37) (end 183.65 93.27) (width 0.2) (layer "F.Cu") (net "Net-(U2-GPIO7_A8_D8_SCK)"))
 (segment (start 189.185635 94.37) (end 184.75 94.37) (width 0.2) (layer "F.Cu") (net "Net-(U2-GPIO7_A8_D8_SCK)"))
 (segment (start 197.62 85.08) (end 189.83 92.87) (width 0.2) (layer "F.Cu") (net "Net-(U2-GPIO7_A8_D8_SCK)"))
 (segment (start 197.62 80) (end 186.19 91.43) (width 0.2) (layer "F.Cu") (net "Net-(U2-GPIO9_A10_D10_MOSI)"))
 (segment (start 186.19 91.43) (end 186.19 93.27) (width 0.2) (layer "F.Cu") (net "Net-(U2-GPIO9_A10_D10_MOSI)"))
 (segment (start 209.0875 93) (end 209.835 92.2525) (width 0.2) (layer "B.Cu") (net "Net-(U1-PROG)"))
 (segment (start 209.835 92.2525) (end 209.835 89.775) (width 0.2) (layer "B.Cu") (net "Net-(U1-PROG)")))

